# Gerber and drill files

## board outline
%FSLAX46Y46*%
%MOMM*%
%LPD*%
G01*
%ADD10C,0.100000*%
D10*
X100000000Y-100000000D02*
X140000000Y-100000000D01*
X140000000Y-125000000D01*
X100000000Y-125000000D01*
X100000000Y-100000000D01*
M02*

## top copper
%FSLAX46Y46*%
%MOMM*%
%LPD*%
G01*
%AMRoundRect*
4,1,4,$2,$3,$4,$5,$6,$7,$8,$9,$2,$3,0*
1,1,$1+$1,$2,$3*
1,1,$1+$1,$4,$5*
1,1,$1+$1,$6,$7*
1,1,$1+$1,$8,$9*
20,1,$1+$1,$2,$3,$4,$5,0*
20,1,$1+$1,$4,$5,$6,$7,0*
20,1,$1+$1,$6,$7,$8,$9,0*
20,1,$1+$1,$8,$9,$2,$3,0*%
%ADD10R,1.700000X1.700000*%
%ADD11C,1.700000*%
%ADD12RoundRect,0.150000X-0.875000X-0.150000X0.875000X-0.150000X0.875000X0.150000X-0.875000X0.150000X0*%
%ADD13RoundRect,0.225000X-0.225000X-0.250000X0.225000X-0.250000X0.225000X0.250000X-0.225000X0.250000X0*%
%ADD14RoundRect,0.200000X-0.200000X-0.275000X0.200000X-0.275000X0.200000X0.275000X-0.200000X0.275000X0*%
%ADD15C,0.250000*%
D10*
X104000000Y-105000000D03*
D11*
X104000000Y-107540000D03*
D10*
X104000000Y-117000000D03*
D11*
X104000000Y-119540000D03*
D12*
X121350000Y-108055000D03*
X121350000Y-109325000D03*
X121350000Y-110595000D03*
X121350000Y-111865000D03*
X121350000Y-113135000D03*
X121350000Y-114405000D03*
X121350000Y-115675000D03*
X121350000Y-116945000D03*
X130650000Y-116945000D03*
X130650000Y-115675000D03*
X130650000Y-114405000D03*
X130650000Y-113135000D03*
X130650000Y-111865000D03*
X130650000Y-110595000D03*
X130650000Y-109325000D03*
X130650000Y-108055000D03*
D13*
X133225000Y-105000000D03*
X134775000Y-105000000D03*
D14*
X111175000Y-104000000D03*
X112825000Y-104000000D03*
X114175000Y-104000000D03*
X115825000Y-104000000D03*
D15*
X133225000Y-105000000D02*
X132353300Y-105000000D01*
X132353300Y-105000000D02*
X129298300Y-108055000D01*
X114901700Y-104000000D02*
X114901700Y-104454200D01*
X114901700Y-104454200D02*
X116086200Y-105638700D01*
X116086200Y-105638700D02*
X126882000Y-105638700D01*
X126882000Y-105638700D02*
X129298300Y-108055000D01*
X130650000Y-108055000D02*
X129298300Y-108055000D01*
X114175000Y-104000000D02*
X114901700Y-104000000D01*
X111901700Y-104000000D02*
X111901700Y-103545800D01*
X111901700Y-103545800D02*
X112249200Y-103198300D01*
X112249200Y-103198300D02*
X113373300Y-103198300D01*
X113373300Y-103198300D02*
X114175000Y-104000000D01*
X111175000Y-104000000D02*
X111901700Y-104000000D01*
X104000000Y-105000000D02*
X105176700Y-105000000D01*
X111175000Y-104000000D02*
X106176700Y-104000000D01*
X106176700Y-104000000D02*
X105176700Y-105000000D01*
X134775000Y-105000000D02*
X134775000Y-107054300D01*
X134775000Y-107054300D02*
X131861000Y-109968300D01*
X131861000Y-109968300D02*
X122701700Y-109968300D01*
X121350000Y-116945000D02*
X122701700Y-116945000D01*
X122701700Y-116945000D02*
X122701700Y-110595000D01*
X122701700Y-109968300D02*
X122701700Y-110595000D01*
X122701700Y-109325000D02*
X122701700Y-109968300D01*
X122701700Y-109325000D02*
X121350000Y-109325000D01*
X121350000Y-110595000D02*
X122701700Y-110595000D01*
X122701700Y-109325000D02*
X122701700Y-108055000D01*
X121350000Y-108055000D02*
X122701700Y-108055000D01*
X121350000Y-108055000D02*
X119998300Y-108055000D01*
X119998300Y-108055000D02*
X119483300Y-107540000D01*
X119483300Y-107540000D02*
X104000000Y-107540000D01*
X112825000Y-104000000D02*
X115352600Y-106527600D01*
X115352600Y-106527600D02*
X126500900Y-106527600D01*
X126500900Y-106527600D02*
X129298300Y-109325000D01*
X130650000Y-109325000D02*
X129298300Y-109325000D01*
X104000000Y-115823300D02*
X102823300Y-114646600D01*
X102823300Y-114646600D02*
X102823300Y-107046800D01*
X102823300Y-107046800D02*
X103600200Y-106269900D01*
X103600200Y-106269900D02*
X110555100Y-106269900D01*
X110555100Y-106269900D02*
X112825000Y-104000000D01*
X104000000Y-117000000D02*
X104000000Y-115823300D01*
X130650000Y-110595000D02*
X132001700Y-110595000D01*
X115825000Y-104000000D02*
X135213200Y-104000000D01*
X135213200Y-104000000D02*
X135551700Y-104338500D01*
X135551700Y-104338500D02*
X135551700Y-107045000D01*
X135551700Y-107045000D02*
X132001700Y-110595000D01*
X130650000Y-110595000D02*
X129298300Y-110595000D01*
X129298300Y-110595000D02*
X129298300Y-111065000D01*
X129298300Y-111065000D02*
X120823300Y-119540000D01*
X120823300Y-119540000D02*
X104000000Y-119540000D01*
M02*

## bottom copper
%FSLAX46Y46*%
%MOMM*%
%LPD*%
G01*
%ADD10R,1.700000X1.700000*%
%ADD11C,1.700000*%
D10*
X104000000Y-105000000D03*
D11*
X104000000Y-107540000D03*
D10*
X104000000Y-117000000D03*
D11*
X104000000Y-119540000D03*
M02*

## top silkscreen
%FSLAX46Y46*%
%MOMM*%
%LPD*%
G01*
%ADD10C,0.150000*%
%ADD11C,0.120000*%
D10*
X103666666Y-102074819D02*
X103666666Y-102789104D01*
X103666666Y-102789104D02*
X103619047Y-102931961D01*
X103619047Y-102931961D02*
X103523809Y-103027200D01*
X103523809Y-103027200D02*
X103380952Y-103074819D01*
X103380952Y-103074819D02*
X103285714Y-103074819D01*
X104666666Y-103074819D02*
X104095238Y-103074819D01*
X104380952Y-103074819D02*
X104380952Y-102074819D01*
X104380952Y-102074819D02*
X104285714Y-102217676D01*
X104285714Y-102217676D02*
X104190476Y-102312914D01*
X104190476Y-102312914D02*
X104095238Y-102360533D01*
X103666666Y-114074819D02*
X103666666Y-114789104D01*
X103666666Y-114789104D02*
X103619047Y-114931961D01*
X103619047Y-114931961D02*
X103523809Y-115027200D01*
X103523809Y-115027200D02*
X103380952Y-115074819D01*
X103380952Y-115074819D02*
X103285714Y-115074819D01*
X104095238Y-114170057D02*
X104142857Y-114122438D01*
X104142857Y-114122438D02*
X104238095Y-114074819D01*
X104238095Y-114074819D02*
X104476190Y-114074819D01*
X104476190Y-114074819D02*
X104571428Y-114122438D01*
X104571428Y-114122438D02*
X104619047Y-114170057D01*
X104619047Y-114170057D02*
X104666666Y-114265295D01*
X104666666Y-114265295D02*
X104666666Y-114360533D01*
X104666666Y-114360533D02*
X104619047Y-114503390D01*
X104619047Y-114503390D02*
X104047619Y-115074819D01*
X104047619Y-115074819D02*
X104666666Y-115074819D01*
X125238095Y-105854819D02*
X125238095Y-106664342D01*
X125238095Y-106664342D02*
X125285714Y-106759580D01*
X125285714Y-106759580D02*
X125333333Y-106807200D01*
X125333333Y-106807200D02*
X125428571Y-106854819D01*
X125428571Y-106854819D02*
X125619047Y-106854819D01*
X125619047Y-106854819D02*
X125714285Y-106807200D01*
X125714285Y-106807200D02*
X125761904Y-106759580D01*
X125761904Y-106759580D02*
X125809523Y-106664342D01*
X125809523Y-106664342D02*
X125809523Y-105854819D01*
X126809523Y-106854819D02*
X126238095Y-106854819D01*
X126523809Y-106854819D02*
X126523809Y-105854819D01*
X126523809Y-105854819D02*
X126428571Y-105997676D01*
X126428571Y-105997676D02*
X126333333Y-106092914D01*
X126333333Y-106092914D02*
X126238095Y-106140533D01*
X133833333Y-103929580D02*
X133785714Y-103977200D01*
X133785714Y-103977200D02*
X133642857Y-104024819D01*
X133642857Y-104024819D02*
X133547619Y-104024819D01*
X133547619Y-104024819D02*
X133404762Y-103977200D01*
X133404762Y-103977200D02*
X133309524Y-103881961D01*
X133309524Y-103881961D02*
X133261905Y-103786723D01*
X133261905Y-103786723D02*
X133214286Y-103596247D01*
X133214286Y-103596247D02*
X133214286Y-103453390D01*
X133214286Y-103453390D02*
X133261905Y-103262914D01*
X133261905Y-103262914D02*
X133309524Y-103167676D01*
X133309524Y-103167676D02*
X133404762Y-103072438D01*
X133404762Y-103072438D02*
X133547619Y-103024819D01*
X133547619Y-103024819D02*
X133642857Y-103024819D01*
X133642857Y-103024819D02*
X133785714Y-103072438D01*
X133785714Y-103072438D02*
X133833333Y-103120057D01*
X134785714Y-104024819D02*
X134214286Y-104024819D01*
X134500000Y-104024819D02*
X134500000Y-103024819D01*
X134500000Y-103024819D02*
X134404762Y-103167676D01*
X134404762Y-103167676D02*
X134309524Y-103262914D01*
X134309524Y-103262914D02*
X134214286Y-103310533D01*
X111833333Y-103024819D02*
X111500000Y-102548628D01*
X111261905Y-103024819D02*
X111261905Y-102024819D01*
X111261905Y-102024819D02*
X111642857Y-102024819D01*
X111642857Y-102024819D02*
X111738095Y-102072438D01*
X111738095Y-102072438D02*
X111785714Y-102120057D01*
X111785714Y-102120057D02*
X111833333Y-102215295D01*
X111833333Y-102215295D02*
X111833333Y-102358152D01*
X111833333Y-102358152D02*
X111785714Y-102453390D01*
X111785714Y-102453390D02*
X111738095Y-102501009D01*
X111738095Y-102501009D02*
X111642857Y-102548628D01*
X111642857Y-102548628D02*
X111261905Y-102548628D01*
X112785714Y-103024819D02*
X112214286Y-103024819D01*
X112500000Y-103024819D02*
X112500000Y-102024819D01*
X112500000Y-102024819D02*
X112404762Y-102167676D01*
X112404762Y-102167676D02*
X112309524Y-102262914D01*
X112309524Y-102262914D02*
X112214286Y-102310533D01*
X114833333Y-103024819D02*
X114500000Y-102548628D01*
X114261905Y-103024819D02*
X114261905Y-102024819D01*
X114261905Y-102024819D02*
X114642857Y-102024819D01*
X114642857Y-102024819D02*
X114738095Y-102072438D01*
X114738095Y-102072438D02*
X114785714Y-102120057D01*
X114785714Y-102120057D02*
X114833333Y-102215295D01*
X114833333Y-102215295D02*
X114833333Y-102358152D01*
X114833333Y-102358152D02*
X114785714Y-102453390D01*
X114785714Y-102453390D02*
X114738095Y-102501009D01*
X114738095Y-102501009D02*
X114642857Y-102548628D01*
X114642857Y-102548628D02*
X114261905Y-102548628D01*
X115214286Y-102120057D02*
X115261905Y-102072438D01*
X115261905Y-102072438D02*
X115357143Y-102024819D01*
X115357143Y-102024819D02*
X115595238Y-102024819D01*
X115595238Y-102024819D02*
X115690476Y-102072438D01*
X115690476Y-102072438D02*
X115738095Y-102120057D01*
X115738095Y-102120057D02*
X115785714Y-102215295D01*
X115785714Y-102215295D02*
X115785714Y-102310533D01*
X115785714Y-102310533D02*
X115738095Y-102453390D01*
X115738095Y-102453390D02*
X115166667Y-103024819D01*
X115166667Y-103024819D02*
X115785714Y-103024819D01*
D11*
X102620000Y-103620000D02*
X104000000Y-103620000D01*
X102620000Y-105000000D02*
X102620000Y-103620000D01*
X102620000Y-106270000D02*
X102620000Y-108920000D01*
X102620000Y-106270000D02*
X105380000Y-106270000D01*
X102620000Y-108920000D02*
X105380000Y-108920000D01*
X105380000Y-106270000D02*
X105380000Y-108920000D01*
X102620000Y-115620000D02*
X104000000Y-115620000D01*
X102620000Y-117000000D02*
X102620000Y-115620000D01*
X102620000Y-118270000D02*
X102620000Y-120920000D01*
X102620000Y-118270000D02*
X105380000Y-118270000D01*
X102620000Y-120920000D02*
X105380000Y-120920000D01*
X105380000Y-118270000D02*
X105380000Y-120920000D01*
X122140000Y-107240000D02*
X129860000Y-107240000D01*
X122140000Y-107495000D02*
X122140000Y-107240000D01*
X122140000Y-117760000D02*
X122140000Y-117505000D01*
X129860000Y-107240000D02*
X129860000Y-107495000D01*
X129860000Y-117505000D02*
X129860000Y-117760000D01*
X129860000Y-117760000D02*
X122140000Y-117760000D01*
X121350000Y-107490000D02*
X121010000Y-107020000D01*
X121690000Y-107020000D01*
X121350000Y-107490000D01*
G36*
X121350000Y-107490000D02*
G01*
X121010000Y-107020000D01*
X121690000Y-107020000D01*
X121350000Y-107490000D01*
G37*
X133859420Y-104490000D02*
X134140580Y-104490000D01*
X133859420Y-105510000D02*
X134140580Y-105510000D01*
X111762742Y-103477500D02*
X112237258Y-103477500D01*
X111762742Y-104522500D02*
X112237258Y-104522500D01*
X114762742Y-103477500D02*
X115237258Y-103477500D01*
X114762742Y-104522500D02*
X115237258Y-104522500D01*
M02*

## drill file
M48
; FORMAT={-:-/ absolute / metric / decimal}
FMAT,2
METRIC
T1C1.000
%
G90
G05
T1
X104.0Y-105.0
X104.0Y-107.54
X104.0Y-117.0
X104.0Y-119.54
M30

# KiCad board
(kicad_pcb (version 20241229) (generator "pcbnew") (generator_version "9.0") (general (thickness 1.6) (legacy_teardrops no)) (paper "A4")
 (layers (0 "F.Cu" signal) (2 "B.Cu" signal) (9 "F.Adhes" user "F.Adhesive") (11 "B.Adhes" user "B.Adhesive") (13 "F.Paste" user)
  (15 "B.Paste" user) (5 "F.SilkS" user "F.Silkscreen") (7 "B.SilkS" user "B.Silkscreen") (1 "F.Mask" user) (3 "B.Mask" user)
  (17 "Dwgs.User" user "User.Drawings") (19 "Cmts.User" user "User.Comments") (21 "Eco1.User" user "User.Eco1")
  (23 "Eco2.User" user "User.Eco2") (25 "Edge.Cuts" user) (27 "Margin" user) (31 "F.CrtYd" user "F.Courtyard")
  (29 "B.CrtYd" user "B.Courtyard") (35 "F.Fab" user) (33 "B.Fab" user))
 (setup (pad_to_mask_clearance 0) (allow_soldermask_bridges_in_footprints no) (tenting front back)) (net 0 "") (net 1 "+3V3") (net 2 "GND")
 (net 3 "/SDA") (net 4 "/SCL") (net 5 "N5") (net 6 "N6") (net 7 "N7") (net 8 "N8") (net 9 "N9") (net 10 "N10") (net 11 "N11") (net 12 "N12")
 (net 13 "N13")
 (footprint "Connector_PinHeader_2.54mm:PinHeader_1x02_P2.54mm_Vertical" (layer "F.Cu") (at 104 105)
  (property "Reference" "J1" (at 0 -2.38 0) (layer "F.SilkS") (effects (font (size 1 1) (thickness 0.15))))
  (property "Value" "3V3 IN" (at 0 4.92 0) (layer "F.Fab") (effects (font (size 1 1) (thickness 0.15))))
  (fp_line (start -1.38 -1.38) (end 0 -1.38) (stroke (width 0.12) (type solid)) (layer "F.SilkS"))
  (fp_line (start -1.38 0) (end -1.38 -1.38) (stroke (width 0.12) (type solid)) (layer "F.SilkS"))
  (fp_line (start -1.38 1.27) (end -1.38 3.92) (stroke (width 0.12) (type solid)) (layer "F.SilkS"))
  (fp_line (start -1.38 1.27) (end 1.38 1.27) (stroke (width 0.12) (type solid)) (layer "F.SilkS"))
  (fp_line (start -1.38 3.92) (end 1.38 3.92) (stroke (width 0.12) (type solid)) (layer "F.SilkS"))
  (fp_line (start 1.38 1.27) (end 1.38 3.92) (stroke (width 0.12) (type solid)) (layer "F.SilkS"))
  (pad "1" thru_hole rect (at 0 0) (size 1.7 1.7) (drill 1) (layers "*.Cu" "*.Mask") (remove_unused_layers no) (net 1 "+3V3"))
  (pad "2" thru_hole circle (at 0 2.54) (size 1.7 1.7) (drill 1) (layers "*.Cu" "*.Mask") (remove_unused_layers no) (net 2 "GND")))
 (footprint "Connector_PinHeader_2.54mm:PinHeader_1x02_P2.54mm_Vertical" (layer "F.Cu") (at 104 117)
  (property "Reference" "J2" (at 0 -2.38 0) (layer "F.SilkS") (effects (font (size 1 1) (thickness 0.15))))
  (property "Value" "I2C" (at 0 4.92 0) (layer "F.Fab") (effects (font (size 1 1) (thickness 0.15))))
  (fp_line (start -1.38 -1.38) (end 0 -1.38) (stroke (width 0.12) (type solid)) (layer "F.SilkS"))
  (fp_line (start -1.38 0) (end -1.38 -1.38) (stroke (width 0.12) (type solid)) (layer "F.SilkS"))
  (fp_line (start -1.38 1.27) (end -1.38 3.92) (stroke (width 0.12) (type solid)) (layer "F.SilkS"))
  (fp_line (start -1.38 1.27) (end 1.38 1.27) (stroke (width 0.12) (type solid)) (layer "F.SilkS"))
  (fp_line (start -1.38 3.92) (end 1.38 3.92) (stroke (width 0.12) (type solid)) (layer "F.SilkS"))
  (fp_line (start 1.38 1.27) (end 1.38 3.92) (stroke (width 0.12) (type solid)) (layer "F.SilkS"))
  (pad "1" thru_hole rect (at 0 0) (size 1.7 1.7) (drill 1) (layers "*.Cu" "*.Mask") (remove_unused_layers no) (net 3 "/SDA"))
  (pad "2" thru_hole circle (at 0 2.54) (size 1.7 1.7) (drill 1) (layers "*.Cu" "*.Mask") (remove_unused_layers no) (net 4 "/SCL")))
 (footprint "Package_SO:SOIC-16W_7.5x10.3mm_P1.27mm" (layer "F.Cu") (at 126 112.5)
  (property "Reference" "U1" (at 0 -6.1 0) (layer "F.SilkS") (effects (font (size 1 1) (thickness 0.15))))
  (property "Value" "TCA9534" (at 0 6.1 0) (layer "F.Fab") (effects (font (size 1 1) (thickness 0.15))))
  (fp_line (start -3.86 -5.26) (end 3.86 -5.26) (stroke (width 0.12) (type solid)) (layer "F.SilkS"))
  (fp_line (start -3.86 -5.005) (end -3.86 -5.26) (stroke (width 0.12) (type solid)) (layer "F.SilkS"))
  (fp_line (start -3.86 5.26) (end -3.86 5.005) (stroke (width 0.12) (type solid)) (layer "F.SilkS"))
  (fp_line (start 3.86 -5.26) (end 3.86 -5.005) (stroke (width 0.12) (type solid)) (layer "F.SilkS"))
  (fp_line (start 3.86 5.005) (end 3.86 5.26) (stroke (width 0.12) (type solid)) (layer "F.SilkS"))
  (fp_line (start 3.86 5.26) (end -3.86 5.26) (stroke (width 0.12) (type solid)) (layer "F.SilkS"))
  (fp_poly (pts (xy -4.65 -5.01) (xy -4.99 -5.48) (xy -4.31 -5.48)) (stroke (width 0.12) (type solid)) (fill yes) (layer "F.SilkS"))
  (pad "1" smd roundrect (at -4.65 -4.445) (size 2.05 0.6) (layers "F.Cu" "F.Mask" "F.Paste") (roundrect_rratio 0.25) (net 2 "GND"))
  (pad "2" smd roundrect (at -4.65 -3.175) (size 2.05 0.6) (layers "F.Cu" "F.Mask" "F.Paste") (roundrect_rratio 0.25) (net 2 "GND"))
  (pad "3" smd roundrect (at -4.65 -1.905) (size 2.05 0.6) (layers "F.Cu" "F.Mask" "F.Paste") (roundrect_rratio 0.25) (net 2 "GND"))
  (pad "4" smd roundrect (at -4.65 -0.635) (size 2.05 0.6) (layers "F.Cu" "F.Mask" "F.Paste") (roundrect_rratio 0.25) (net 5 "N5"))
  (pad "5" smd roundrect (at -4.65 0.635) (size 2.05 0.6) (layers "F.Cu" "F.Mask" "F.Paste") (roundrect_rratio 0.25) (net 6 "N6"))
  (pad "6" smd roundrect (at -4.65 1.905) (size 2.05 0.6) (layers "F.Cu" "F.Mask" "F.Paste") (roundrect_rratio 0.25) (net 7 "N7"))
  (pad "7" smd roundrect (at -4.65 3.175) (size 2.05 0.6) (layers "F.Cu" "F.Mask" "F.Paste") (roundrect_rratio 0.25) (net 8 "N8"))
  (pad "8" smd roundrect (at -4.65 4.445) (size 2.05 0.6) (layers "F.Cu" "F.Mask" "F.Paste") (roundrect_rratio 0.25) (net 2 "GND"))
  (pad "9" smd roundrect (at 4.65 4.445) (size 2.05 0.6) (layers "F.Cu" "F.Mask" "F.Paste") (roundrect_rratio 0.25) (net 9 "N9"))
  (pad "10" smd roundrect (at 4.65 3.175) (size 2.05 0.6) (layers "F.Cu" "F.Mask" "F.Paste") (roundrect_rratio 0.25) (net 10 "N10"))
  (pad "11" smd roundrect (at 4.65 1.905) (size 2.05 0.6) (layers "F.Cu" "F.Mask" "F.Paste") (roundrect_rratio 0.25) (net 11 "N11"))
  (pad "12" smd roundrect (at 4.65 0.635) (size 2.05 0.6) (layers "F.Cu" "F.Mask" "F.Paste") (roundrect_rratio 0.25) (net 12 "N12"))
  (pad "13" smd roundrect (at 4.65 -0.635) (size 2.05 0.6) (layers "F.Cu" "F.Mask" "F.Paste") (roundrect_rratio 0.25) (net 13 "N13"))
  (pad "14" smd roundrect (at 4.65 -1.905) (size 2.05 0.6) (layers "F.Cu" "F.Mask" "F.Paste") (roundrect_rratio 0.25) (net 4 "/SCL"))
  (pad "15" smd roundrect (at 4.65 -3.175) (size 2.05 0.6) (layers "F.Cu" "F.Mask" "F.Paste") (roundrect_rratio 0.25) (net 3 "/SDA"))
  (pad "16" smd roundrect (at 4.65 -4.445) (size 2.05 0.6) (layers "F.Cu" "F.Mask" "F.Paste") (roundrect_rratio 0.25) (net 1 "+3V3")))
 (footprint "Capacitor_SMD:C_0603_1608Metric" (layer "F.Cu") (at 134 105)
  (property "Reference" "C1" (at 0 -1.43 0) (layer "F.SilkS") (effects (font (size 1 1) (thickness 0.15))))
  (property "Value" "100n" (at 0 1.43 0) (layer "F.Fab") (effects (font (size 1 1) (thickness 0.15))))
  (fp_line (start -0.14058 -0.51) (end 0.14058 -0.51) (stroke (width 0.12) (type solid)) (layer "F.SilkS"))
  (fp_line (start -0.14058 0.51) (end 0.14058 0.51) (stroke (width 0.12) (type solid)) (layer "F.SilkS"))
  (pad "1" smd roundrect (at -0.775 0) (size 0.9 0.95) (layers "F.Cu" "F.Mask" "F.Paste") (roundrect_rratio 0.25) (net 1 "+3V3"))
  (pad "2" smd roundrect (at 0.775 0) (size 0.9 0.95) (layers "F.Cu" "F.Mask" "F.Paste") (roundrect_rratio 0.25) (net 2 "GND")))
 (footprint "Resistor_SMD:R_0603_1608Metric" (layer "F.Cu") (at 112 104)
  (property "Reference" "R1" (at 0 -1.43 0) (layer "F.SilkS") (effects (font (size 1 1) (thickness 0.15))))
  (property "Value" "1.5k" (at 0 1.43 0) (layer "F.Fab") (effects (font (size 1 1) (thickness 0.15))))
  (fp_line (start -0.237258 -0.5225) (end 0.237258 -0.5225) (stroke (width 0.12) (type solid)) (layer "F.SilkS"))
  (fp_line (start -0.237258 0.5225) (end 0.237258 0.5225) (stroke (width 0.12) (type solid)) (layer "F.SilkS"))
  (pad "1" smd roundrect (at -0.825 0) (size 0.8 0.95) (layers "F.Cu" "F.Mask" "F.Paste") (roundrect_rratio 0.25) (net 1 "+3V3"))
  (pad "2" smd roundrect (at 0.825 0) (size 0.8 0.95) (layers "F.Cu" "F.Mask" "F.Paste") (roundrect_rratio 0.25) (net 3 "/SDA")))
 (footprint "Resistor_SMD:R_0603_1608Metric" (layer "F.Cu") (at 115 104)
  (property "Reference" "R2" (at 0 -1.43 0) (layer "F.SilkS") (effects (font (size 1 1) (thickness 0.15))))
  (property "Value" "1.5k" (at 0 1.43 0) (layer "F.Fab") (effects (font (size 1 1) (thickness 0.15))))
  (fp_line (start -0.237258 -0.5225) (end 0.237258 -0.5225) (stroke (width 0.12) (type solid)) (layer "F.SilkS"))
  (fp_line (start -0.237258 0.5225) (end 0.237258 0.5225) (stroke (width 0.12) (type solid)) (layer "F.SilkS"))
  (pad "1" smd roundrect (at -0.825 0) (size 0.8 0.95) (layers "F.Cu" "F.Mask" "F.Paste") (roundrect_rratio 0.25) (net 1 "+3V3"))
  (pad "2" smd roundrect (at 0.825 0) (size 0.8 0.95) (layers "F.Cu" "F.Mask" "F.Paste") (roundrect_rratio 0.25) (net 4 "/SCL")))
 (gr_rect (start 100 100) (end 140 125) (stroke (width 0.1) (type default)) (fill no) (layer "Edge.Cuts"))
 (segment (start 133.225 105) (end 132.3533 105) (width 0.25) (layer "F.Cu") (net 1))
 (segment (start 132.3533 105) (end 129.2983 108.055) (width 0.25) (layer "F.Cu") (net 1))
 (segment (start 114.9017 104) (end 114.9017 104.4542) (width 0.25) (layer "F.Cu") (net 1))
 (segment (start 114.9017 104.4542) (end 116.0862 105.6387) (width 0.25) (layer "F.Cu") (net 1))
 (segment (start 116.0862 105.6387) (end 126.882 105.6387) (width 0.25) (layer "F.Cu") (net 1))
 (segment (start 126.882 105.6387) (end 129.2983 108.055) (width 0.25) (layer "F.Cu") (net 1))
 (segment (start 130.65 108.055) (end 129.2983 108.055) (width 0.25) (layer "F.Cu") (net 1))
 (segment (start 114.175 104) (end 114.9017 104) (width 0.25) (layer "F.Cu") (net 1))
 (segment (start 111.9017 104) (end 111.9017 103.5458) (width 0.25) (layer "F.Cu") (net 1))
 (segment (start 111.9017 103.5458) (end 112.2492 103.1983) (width 0.25) (layer "F.Cu") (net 1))
 (segment (start 112.2492 103.1983) (end 113.3733 103.1983) (width 0.25) (layer "F.Cu") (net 1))
 (segment (start 113.3733 103.1983) (end 114.175 104) (width 0.25) (layer "F.Cu") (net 1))
 (segment (start 111.175 104) (end 111.9017 104) (width 0.25) (layer "F.Cu") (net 1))
 (segment (start 104 105) (end 105.1767 105) (width 0.25) (layer "F.Cu") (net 1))
 (segment (start 111.175 104) (end 106.1767 104) (width 0.25) (layer "F.Cu") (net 1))
 (segment (start 106.1767 104) (end 105.1767 105) (width 0.25) (layer "F.Cu") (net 1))
 (segment (start 134.775 105) (end 134.775 107.0543) (width 0.25) (layer "F.Cu") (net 2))
 (segment (start 134.775 107.0543) (end 131.861 109.9683) (width 0.25) (layer "F.Cu") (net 2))
 (segment (start 131.861 109.9683) (end 122.7017 109.9683) (width 0.25) (layer "F.Cu") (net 2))
 (segment (start 121.35 116.945) (end 122.7017 116.945) (width 0.25) (layer "F.Cu") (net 2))
 (segment (start 122.7017 116.945) (end 122.7017 110.595) (width 0.25) (layer "F.Cu") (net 2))
 (segment (start 122.7017 109.9683) (end 122.7017 110.595) (width 0.25) (layer "F.Cu") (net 2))
 (segment (start 122.7017 109.325) (end 122.7017 109.9683) (width 0.25) (layer "F.Cu") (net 2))
 (segment (start 122.7017 109.325) (end 121.35 109.325) (width 0.25) (layer "F.Cu") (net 2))
 (segment (start 121.35 110.595) (end 122.7017 110.595) (width 0.25) (layer "F.Cu") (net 2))
 (segment (start 122.7017 109.325) (end 122.7017 108.055) (width 0.25) (layer "F.Cu") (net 2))
 (segment (start 121.35 108.055) (end 122.7017 108.055) (width 0.25) (layer "F.Cu") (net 2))
 (segment (start 121.35 108.055) (end 119.9983 108.055) (width 0.25) (layer "F.Cu") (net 2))
 (segment (start 119.9983 108.055) (end 119.4833 107.54) (width 0.25) (layer "F.Cu") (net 2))
 (segment (start 119.4833 107.54) (end 104 107.54) (width 0.25) (layer "F.Cu") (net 2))
 (segment (start 112.825 104) (end 115.3526 106.5276) (width 0.25) (layer "F.Cu") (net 3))
 (segment (start 115.3526 106.5276) (end 126.5009 106.5276) (width 0.25) (layer "F.Cu") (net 3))
 (segment (start 126.5009 106.5276) (end 129.2983 109.325) (width 0.25) (layer "F.Cu") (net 3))
 (segment (start 130.65 109.325) (end 129.2983 109.325) (width 0.25) (layer "F.Cu") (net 3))
 (segment (start 104 115.8233) (end 102.8233 114.6466) (width 0.25) (layer "F.Cu") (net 3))
 (segment (start 102.8233 114.6466) (end 102.8233 107.0468) (width 0.25) (layer "F.Cu") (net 3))
 (segment (start 102.8233 107.0468) (end 103.6002 106.2699) (width 0.25) (layer "F.Cu") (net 3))
 (segment (start 103.6002 106.2699) (end 110.5551 106.2699) (width 0.25) (layer "F.Cu") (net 3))
 (segment (start 110.5551 106.2699) (end 112.825 104) (width 0.25) (layer "F.Cu") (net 3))
 (segment (start 104 117) (end 104 115.8233) (width 0.25) (layer "F.Cu") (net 3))
 (segment (start 130.65 110.595) (end 132.0017 110.595) (width 0.25) (layer "F.Cu") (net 4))
 (segment (start 115.825 104) (end 135.2132 104) (width 0.25) (layer "F.Cu") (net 4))
 (segment (start 135.2132 104) (end 135.5517 104.3385) (width 0.25) (layer "F.Cu") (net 4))
 (segment (start 135.5517 104.3385) (end 135.5517 107.045) (width 0.25) (layer "F.Cu") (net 4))
 (segment (start 135.5517 107.045) (end 132.0017 110.595) (width 0.25) (layer "F.Cu") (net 4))
 (segment (start 130.65 110.595) (end 129.2983 110.595) (width 0.25) (layer "F.Cu") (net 4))
 (segment (start 129.2983 110.595) (end 129.2983 111.065) (width 0.25) (layer "F.Cu") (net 4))
 (segment (start 129.2983 111.065) (end 120.8233 119.54) (width 0.25) (layer "F.Cu") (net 4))
 (segment (start 120.8233 119.54) (end 104 119.54) (width 0.25) (layer "F.Cu") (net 4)))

